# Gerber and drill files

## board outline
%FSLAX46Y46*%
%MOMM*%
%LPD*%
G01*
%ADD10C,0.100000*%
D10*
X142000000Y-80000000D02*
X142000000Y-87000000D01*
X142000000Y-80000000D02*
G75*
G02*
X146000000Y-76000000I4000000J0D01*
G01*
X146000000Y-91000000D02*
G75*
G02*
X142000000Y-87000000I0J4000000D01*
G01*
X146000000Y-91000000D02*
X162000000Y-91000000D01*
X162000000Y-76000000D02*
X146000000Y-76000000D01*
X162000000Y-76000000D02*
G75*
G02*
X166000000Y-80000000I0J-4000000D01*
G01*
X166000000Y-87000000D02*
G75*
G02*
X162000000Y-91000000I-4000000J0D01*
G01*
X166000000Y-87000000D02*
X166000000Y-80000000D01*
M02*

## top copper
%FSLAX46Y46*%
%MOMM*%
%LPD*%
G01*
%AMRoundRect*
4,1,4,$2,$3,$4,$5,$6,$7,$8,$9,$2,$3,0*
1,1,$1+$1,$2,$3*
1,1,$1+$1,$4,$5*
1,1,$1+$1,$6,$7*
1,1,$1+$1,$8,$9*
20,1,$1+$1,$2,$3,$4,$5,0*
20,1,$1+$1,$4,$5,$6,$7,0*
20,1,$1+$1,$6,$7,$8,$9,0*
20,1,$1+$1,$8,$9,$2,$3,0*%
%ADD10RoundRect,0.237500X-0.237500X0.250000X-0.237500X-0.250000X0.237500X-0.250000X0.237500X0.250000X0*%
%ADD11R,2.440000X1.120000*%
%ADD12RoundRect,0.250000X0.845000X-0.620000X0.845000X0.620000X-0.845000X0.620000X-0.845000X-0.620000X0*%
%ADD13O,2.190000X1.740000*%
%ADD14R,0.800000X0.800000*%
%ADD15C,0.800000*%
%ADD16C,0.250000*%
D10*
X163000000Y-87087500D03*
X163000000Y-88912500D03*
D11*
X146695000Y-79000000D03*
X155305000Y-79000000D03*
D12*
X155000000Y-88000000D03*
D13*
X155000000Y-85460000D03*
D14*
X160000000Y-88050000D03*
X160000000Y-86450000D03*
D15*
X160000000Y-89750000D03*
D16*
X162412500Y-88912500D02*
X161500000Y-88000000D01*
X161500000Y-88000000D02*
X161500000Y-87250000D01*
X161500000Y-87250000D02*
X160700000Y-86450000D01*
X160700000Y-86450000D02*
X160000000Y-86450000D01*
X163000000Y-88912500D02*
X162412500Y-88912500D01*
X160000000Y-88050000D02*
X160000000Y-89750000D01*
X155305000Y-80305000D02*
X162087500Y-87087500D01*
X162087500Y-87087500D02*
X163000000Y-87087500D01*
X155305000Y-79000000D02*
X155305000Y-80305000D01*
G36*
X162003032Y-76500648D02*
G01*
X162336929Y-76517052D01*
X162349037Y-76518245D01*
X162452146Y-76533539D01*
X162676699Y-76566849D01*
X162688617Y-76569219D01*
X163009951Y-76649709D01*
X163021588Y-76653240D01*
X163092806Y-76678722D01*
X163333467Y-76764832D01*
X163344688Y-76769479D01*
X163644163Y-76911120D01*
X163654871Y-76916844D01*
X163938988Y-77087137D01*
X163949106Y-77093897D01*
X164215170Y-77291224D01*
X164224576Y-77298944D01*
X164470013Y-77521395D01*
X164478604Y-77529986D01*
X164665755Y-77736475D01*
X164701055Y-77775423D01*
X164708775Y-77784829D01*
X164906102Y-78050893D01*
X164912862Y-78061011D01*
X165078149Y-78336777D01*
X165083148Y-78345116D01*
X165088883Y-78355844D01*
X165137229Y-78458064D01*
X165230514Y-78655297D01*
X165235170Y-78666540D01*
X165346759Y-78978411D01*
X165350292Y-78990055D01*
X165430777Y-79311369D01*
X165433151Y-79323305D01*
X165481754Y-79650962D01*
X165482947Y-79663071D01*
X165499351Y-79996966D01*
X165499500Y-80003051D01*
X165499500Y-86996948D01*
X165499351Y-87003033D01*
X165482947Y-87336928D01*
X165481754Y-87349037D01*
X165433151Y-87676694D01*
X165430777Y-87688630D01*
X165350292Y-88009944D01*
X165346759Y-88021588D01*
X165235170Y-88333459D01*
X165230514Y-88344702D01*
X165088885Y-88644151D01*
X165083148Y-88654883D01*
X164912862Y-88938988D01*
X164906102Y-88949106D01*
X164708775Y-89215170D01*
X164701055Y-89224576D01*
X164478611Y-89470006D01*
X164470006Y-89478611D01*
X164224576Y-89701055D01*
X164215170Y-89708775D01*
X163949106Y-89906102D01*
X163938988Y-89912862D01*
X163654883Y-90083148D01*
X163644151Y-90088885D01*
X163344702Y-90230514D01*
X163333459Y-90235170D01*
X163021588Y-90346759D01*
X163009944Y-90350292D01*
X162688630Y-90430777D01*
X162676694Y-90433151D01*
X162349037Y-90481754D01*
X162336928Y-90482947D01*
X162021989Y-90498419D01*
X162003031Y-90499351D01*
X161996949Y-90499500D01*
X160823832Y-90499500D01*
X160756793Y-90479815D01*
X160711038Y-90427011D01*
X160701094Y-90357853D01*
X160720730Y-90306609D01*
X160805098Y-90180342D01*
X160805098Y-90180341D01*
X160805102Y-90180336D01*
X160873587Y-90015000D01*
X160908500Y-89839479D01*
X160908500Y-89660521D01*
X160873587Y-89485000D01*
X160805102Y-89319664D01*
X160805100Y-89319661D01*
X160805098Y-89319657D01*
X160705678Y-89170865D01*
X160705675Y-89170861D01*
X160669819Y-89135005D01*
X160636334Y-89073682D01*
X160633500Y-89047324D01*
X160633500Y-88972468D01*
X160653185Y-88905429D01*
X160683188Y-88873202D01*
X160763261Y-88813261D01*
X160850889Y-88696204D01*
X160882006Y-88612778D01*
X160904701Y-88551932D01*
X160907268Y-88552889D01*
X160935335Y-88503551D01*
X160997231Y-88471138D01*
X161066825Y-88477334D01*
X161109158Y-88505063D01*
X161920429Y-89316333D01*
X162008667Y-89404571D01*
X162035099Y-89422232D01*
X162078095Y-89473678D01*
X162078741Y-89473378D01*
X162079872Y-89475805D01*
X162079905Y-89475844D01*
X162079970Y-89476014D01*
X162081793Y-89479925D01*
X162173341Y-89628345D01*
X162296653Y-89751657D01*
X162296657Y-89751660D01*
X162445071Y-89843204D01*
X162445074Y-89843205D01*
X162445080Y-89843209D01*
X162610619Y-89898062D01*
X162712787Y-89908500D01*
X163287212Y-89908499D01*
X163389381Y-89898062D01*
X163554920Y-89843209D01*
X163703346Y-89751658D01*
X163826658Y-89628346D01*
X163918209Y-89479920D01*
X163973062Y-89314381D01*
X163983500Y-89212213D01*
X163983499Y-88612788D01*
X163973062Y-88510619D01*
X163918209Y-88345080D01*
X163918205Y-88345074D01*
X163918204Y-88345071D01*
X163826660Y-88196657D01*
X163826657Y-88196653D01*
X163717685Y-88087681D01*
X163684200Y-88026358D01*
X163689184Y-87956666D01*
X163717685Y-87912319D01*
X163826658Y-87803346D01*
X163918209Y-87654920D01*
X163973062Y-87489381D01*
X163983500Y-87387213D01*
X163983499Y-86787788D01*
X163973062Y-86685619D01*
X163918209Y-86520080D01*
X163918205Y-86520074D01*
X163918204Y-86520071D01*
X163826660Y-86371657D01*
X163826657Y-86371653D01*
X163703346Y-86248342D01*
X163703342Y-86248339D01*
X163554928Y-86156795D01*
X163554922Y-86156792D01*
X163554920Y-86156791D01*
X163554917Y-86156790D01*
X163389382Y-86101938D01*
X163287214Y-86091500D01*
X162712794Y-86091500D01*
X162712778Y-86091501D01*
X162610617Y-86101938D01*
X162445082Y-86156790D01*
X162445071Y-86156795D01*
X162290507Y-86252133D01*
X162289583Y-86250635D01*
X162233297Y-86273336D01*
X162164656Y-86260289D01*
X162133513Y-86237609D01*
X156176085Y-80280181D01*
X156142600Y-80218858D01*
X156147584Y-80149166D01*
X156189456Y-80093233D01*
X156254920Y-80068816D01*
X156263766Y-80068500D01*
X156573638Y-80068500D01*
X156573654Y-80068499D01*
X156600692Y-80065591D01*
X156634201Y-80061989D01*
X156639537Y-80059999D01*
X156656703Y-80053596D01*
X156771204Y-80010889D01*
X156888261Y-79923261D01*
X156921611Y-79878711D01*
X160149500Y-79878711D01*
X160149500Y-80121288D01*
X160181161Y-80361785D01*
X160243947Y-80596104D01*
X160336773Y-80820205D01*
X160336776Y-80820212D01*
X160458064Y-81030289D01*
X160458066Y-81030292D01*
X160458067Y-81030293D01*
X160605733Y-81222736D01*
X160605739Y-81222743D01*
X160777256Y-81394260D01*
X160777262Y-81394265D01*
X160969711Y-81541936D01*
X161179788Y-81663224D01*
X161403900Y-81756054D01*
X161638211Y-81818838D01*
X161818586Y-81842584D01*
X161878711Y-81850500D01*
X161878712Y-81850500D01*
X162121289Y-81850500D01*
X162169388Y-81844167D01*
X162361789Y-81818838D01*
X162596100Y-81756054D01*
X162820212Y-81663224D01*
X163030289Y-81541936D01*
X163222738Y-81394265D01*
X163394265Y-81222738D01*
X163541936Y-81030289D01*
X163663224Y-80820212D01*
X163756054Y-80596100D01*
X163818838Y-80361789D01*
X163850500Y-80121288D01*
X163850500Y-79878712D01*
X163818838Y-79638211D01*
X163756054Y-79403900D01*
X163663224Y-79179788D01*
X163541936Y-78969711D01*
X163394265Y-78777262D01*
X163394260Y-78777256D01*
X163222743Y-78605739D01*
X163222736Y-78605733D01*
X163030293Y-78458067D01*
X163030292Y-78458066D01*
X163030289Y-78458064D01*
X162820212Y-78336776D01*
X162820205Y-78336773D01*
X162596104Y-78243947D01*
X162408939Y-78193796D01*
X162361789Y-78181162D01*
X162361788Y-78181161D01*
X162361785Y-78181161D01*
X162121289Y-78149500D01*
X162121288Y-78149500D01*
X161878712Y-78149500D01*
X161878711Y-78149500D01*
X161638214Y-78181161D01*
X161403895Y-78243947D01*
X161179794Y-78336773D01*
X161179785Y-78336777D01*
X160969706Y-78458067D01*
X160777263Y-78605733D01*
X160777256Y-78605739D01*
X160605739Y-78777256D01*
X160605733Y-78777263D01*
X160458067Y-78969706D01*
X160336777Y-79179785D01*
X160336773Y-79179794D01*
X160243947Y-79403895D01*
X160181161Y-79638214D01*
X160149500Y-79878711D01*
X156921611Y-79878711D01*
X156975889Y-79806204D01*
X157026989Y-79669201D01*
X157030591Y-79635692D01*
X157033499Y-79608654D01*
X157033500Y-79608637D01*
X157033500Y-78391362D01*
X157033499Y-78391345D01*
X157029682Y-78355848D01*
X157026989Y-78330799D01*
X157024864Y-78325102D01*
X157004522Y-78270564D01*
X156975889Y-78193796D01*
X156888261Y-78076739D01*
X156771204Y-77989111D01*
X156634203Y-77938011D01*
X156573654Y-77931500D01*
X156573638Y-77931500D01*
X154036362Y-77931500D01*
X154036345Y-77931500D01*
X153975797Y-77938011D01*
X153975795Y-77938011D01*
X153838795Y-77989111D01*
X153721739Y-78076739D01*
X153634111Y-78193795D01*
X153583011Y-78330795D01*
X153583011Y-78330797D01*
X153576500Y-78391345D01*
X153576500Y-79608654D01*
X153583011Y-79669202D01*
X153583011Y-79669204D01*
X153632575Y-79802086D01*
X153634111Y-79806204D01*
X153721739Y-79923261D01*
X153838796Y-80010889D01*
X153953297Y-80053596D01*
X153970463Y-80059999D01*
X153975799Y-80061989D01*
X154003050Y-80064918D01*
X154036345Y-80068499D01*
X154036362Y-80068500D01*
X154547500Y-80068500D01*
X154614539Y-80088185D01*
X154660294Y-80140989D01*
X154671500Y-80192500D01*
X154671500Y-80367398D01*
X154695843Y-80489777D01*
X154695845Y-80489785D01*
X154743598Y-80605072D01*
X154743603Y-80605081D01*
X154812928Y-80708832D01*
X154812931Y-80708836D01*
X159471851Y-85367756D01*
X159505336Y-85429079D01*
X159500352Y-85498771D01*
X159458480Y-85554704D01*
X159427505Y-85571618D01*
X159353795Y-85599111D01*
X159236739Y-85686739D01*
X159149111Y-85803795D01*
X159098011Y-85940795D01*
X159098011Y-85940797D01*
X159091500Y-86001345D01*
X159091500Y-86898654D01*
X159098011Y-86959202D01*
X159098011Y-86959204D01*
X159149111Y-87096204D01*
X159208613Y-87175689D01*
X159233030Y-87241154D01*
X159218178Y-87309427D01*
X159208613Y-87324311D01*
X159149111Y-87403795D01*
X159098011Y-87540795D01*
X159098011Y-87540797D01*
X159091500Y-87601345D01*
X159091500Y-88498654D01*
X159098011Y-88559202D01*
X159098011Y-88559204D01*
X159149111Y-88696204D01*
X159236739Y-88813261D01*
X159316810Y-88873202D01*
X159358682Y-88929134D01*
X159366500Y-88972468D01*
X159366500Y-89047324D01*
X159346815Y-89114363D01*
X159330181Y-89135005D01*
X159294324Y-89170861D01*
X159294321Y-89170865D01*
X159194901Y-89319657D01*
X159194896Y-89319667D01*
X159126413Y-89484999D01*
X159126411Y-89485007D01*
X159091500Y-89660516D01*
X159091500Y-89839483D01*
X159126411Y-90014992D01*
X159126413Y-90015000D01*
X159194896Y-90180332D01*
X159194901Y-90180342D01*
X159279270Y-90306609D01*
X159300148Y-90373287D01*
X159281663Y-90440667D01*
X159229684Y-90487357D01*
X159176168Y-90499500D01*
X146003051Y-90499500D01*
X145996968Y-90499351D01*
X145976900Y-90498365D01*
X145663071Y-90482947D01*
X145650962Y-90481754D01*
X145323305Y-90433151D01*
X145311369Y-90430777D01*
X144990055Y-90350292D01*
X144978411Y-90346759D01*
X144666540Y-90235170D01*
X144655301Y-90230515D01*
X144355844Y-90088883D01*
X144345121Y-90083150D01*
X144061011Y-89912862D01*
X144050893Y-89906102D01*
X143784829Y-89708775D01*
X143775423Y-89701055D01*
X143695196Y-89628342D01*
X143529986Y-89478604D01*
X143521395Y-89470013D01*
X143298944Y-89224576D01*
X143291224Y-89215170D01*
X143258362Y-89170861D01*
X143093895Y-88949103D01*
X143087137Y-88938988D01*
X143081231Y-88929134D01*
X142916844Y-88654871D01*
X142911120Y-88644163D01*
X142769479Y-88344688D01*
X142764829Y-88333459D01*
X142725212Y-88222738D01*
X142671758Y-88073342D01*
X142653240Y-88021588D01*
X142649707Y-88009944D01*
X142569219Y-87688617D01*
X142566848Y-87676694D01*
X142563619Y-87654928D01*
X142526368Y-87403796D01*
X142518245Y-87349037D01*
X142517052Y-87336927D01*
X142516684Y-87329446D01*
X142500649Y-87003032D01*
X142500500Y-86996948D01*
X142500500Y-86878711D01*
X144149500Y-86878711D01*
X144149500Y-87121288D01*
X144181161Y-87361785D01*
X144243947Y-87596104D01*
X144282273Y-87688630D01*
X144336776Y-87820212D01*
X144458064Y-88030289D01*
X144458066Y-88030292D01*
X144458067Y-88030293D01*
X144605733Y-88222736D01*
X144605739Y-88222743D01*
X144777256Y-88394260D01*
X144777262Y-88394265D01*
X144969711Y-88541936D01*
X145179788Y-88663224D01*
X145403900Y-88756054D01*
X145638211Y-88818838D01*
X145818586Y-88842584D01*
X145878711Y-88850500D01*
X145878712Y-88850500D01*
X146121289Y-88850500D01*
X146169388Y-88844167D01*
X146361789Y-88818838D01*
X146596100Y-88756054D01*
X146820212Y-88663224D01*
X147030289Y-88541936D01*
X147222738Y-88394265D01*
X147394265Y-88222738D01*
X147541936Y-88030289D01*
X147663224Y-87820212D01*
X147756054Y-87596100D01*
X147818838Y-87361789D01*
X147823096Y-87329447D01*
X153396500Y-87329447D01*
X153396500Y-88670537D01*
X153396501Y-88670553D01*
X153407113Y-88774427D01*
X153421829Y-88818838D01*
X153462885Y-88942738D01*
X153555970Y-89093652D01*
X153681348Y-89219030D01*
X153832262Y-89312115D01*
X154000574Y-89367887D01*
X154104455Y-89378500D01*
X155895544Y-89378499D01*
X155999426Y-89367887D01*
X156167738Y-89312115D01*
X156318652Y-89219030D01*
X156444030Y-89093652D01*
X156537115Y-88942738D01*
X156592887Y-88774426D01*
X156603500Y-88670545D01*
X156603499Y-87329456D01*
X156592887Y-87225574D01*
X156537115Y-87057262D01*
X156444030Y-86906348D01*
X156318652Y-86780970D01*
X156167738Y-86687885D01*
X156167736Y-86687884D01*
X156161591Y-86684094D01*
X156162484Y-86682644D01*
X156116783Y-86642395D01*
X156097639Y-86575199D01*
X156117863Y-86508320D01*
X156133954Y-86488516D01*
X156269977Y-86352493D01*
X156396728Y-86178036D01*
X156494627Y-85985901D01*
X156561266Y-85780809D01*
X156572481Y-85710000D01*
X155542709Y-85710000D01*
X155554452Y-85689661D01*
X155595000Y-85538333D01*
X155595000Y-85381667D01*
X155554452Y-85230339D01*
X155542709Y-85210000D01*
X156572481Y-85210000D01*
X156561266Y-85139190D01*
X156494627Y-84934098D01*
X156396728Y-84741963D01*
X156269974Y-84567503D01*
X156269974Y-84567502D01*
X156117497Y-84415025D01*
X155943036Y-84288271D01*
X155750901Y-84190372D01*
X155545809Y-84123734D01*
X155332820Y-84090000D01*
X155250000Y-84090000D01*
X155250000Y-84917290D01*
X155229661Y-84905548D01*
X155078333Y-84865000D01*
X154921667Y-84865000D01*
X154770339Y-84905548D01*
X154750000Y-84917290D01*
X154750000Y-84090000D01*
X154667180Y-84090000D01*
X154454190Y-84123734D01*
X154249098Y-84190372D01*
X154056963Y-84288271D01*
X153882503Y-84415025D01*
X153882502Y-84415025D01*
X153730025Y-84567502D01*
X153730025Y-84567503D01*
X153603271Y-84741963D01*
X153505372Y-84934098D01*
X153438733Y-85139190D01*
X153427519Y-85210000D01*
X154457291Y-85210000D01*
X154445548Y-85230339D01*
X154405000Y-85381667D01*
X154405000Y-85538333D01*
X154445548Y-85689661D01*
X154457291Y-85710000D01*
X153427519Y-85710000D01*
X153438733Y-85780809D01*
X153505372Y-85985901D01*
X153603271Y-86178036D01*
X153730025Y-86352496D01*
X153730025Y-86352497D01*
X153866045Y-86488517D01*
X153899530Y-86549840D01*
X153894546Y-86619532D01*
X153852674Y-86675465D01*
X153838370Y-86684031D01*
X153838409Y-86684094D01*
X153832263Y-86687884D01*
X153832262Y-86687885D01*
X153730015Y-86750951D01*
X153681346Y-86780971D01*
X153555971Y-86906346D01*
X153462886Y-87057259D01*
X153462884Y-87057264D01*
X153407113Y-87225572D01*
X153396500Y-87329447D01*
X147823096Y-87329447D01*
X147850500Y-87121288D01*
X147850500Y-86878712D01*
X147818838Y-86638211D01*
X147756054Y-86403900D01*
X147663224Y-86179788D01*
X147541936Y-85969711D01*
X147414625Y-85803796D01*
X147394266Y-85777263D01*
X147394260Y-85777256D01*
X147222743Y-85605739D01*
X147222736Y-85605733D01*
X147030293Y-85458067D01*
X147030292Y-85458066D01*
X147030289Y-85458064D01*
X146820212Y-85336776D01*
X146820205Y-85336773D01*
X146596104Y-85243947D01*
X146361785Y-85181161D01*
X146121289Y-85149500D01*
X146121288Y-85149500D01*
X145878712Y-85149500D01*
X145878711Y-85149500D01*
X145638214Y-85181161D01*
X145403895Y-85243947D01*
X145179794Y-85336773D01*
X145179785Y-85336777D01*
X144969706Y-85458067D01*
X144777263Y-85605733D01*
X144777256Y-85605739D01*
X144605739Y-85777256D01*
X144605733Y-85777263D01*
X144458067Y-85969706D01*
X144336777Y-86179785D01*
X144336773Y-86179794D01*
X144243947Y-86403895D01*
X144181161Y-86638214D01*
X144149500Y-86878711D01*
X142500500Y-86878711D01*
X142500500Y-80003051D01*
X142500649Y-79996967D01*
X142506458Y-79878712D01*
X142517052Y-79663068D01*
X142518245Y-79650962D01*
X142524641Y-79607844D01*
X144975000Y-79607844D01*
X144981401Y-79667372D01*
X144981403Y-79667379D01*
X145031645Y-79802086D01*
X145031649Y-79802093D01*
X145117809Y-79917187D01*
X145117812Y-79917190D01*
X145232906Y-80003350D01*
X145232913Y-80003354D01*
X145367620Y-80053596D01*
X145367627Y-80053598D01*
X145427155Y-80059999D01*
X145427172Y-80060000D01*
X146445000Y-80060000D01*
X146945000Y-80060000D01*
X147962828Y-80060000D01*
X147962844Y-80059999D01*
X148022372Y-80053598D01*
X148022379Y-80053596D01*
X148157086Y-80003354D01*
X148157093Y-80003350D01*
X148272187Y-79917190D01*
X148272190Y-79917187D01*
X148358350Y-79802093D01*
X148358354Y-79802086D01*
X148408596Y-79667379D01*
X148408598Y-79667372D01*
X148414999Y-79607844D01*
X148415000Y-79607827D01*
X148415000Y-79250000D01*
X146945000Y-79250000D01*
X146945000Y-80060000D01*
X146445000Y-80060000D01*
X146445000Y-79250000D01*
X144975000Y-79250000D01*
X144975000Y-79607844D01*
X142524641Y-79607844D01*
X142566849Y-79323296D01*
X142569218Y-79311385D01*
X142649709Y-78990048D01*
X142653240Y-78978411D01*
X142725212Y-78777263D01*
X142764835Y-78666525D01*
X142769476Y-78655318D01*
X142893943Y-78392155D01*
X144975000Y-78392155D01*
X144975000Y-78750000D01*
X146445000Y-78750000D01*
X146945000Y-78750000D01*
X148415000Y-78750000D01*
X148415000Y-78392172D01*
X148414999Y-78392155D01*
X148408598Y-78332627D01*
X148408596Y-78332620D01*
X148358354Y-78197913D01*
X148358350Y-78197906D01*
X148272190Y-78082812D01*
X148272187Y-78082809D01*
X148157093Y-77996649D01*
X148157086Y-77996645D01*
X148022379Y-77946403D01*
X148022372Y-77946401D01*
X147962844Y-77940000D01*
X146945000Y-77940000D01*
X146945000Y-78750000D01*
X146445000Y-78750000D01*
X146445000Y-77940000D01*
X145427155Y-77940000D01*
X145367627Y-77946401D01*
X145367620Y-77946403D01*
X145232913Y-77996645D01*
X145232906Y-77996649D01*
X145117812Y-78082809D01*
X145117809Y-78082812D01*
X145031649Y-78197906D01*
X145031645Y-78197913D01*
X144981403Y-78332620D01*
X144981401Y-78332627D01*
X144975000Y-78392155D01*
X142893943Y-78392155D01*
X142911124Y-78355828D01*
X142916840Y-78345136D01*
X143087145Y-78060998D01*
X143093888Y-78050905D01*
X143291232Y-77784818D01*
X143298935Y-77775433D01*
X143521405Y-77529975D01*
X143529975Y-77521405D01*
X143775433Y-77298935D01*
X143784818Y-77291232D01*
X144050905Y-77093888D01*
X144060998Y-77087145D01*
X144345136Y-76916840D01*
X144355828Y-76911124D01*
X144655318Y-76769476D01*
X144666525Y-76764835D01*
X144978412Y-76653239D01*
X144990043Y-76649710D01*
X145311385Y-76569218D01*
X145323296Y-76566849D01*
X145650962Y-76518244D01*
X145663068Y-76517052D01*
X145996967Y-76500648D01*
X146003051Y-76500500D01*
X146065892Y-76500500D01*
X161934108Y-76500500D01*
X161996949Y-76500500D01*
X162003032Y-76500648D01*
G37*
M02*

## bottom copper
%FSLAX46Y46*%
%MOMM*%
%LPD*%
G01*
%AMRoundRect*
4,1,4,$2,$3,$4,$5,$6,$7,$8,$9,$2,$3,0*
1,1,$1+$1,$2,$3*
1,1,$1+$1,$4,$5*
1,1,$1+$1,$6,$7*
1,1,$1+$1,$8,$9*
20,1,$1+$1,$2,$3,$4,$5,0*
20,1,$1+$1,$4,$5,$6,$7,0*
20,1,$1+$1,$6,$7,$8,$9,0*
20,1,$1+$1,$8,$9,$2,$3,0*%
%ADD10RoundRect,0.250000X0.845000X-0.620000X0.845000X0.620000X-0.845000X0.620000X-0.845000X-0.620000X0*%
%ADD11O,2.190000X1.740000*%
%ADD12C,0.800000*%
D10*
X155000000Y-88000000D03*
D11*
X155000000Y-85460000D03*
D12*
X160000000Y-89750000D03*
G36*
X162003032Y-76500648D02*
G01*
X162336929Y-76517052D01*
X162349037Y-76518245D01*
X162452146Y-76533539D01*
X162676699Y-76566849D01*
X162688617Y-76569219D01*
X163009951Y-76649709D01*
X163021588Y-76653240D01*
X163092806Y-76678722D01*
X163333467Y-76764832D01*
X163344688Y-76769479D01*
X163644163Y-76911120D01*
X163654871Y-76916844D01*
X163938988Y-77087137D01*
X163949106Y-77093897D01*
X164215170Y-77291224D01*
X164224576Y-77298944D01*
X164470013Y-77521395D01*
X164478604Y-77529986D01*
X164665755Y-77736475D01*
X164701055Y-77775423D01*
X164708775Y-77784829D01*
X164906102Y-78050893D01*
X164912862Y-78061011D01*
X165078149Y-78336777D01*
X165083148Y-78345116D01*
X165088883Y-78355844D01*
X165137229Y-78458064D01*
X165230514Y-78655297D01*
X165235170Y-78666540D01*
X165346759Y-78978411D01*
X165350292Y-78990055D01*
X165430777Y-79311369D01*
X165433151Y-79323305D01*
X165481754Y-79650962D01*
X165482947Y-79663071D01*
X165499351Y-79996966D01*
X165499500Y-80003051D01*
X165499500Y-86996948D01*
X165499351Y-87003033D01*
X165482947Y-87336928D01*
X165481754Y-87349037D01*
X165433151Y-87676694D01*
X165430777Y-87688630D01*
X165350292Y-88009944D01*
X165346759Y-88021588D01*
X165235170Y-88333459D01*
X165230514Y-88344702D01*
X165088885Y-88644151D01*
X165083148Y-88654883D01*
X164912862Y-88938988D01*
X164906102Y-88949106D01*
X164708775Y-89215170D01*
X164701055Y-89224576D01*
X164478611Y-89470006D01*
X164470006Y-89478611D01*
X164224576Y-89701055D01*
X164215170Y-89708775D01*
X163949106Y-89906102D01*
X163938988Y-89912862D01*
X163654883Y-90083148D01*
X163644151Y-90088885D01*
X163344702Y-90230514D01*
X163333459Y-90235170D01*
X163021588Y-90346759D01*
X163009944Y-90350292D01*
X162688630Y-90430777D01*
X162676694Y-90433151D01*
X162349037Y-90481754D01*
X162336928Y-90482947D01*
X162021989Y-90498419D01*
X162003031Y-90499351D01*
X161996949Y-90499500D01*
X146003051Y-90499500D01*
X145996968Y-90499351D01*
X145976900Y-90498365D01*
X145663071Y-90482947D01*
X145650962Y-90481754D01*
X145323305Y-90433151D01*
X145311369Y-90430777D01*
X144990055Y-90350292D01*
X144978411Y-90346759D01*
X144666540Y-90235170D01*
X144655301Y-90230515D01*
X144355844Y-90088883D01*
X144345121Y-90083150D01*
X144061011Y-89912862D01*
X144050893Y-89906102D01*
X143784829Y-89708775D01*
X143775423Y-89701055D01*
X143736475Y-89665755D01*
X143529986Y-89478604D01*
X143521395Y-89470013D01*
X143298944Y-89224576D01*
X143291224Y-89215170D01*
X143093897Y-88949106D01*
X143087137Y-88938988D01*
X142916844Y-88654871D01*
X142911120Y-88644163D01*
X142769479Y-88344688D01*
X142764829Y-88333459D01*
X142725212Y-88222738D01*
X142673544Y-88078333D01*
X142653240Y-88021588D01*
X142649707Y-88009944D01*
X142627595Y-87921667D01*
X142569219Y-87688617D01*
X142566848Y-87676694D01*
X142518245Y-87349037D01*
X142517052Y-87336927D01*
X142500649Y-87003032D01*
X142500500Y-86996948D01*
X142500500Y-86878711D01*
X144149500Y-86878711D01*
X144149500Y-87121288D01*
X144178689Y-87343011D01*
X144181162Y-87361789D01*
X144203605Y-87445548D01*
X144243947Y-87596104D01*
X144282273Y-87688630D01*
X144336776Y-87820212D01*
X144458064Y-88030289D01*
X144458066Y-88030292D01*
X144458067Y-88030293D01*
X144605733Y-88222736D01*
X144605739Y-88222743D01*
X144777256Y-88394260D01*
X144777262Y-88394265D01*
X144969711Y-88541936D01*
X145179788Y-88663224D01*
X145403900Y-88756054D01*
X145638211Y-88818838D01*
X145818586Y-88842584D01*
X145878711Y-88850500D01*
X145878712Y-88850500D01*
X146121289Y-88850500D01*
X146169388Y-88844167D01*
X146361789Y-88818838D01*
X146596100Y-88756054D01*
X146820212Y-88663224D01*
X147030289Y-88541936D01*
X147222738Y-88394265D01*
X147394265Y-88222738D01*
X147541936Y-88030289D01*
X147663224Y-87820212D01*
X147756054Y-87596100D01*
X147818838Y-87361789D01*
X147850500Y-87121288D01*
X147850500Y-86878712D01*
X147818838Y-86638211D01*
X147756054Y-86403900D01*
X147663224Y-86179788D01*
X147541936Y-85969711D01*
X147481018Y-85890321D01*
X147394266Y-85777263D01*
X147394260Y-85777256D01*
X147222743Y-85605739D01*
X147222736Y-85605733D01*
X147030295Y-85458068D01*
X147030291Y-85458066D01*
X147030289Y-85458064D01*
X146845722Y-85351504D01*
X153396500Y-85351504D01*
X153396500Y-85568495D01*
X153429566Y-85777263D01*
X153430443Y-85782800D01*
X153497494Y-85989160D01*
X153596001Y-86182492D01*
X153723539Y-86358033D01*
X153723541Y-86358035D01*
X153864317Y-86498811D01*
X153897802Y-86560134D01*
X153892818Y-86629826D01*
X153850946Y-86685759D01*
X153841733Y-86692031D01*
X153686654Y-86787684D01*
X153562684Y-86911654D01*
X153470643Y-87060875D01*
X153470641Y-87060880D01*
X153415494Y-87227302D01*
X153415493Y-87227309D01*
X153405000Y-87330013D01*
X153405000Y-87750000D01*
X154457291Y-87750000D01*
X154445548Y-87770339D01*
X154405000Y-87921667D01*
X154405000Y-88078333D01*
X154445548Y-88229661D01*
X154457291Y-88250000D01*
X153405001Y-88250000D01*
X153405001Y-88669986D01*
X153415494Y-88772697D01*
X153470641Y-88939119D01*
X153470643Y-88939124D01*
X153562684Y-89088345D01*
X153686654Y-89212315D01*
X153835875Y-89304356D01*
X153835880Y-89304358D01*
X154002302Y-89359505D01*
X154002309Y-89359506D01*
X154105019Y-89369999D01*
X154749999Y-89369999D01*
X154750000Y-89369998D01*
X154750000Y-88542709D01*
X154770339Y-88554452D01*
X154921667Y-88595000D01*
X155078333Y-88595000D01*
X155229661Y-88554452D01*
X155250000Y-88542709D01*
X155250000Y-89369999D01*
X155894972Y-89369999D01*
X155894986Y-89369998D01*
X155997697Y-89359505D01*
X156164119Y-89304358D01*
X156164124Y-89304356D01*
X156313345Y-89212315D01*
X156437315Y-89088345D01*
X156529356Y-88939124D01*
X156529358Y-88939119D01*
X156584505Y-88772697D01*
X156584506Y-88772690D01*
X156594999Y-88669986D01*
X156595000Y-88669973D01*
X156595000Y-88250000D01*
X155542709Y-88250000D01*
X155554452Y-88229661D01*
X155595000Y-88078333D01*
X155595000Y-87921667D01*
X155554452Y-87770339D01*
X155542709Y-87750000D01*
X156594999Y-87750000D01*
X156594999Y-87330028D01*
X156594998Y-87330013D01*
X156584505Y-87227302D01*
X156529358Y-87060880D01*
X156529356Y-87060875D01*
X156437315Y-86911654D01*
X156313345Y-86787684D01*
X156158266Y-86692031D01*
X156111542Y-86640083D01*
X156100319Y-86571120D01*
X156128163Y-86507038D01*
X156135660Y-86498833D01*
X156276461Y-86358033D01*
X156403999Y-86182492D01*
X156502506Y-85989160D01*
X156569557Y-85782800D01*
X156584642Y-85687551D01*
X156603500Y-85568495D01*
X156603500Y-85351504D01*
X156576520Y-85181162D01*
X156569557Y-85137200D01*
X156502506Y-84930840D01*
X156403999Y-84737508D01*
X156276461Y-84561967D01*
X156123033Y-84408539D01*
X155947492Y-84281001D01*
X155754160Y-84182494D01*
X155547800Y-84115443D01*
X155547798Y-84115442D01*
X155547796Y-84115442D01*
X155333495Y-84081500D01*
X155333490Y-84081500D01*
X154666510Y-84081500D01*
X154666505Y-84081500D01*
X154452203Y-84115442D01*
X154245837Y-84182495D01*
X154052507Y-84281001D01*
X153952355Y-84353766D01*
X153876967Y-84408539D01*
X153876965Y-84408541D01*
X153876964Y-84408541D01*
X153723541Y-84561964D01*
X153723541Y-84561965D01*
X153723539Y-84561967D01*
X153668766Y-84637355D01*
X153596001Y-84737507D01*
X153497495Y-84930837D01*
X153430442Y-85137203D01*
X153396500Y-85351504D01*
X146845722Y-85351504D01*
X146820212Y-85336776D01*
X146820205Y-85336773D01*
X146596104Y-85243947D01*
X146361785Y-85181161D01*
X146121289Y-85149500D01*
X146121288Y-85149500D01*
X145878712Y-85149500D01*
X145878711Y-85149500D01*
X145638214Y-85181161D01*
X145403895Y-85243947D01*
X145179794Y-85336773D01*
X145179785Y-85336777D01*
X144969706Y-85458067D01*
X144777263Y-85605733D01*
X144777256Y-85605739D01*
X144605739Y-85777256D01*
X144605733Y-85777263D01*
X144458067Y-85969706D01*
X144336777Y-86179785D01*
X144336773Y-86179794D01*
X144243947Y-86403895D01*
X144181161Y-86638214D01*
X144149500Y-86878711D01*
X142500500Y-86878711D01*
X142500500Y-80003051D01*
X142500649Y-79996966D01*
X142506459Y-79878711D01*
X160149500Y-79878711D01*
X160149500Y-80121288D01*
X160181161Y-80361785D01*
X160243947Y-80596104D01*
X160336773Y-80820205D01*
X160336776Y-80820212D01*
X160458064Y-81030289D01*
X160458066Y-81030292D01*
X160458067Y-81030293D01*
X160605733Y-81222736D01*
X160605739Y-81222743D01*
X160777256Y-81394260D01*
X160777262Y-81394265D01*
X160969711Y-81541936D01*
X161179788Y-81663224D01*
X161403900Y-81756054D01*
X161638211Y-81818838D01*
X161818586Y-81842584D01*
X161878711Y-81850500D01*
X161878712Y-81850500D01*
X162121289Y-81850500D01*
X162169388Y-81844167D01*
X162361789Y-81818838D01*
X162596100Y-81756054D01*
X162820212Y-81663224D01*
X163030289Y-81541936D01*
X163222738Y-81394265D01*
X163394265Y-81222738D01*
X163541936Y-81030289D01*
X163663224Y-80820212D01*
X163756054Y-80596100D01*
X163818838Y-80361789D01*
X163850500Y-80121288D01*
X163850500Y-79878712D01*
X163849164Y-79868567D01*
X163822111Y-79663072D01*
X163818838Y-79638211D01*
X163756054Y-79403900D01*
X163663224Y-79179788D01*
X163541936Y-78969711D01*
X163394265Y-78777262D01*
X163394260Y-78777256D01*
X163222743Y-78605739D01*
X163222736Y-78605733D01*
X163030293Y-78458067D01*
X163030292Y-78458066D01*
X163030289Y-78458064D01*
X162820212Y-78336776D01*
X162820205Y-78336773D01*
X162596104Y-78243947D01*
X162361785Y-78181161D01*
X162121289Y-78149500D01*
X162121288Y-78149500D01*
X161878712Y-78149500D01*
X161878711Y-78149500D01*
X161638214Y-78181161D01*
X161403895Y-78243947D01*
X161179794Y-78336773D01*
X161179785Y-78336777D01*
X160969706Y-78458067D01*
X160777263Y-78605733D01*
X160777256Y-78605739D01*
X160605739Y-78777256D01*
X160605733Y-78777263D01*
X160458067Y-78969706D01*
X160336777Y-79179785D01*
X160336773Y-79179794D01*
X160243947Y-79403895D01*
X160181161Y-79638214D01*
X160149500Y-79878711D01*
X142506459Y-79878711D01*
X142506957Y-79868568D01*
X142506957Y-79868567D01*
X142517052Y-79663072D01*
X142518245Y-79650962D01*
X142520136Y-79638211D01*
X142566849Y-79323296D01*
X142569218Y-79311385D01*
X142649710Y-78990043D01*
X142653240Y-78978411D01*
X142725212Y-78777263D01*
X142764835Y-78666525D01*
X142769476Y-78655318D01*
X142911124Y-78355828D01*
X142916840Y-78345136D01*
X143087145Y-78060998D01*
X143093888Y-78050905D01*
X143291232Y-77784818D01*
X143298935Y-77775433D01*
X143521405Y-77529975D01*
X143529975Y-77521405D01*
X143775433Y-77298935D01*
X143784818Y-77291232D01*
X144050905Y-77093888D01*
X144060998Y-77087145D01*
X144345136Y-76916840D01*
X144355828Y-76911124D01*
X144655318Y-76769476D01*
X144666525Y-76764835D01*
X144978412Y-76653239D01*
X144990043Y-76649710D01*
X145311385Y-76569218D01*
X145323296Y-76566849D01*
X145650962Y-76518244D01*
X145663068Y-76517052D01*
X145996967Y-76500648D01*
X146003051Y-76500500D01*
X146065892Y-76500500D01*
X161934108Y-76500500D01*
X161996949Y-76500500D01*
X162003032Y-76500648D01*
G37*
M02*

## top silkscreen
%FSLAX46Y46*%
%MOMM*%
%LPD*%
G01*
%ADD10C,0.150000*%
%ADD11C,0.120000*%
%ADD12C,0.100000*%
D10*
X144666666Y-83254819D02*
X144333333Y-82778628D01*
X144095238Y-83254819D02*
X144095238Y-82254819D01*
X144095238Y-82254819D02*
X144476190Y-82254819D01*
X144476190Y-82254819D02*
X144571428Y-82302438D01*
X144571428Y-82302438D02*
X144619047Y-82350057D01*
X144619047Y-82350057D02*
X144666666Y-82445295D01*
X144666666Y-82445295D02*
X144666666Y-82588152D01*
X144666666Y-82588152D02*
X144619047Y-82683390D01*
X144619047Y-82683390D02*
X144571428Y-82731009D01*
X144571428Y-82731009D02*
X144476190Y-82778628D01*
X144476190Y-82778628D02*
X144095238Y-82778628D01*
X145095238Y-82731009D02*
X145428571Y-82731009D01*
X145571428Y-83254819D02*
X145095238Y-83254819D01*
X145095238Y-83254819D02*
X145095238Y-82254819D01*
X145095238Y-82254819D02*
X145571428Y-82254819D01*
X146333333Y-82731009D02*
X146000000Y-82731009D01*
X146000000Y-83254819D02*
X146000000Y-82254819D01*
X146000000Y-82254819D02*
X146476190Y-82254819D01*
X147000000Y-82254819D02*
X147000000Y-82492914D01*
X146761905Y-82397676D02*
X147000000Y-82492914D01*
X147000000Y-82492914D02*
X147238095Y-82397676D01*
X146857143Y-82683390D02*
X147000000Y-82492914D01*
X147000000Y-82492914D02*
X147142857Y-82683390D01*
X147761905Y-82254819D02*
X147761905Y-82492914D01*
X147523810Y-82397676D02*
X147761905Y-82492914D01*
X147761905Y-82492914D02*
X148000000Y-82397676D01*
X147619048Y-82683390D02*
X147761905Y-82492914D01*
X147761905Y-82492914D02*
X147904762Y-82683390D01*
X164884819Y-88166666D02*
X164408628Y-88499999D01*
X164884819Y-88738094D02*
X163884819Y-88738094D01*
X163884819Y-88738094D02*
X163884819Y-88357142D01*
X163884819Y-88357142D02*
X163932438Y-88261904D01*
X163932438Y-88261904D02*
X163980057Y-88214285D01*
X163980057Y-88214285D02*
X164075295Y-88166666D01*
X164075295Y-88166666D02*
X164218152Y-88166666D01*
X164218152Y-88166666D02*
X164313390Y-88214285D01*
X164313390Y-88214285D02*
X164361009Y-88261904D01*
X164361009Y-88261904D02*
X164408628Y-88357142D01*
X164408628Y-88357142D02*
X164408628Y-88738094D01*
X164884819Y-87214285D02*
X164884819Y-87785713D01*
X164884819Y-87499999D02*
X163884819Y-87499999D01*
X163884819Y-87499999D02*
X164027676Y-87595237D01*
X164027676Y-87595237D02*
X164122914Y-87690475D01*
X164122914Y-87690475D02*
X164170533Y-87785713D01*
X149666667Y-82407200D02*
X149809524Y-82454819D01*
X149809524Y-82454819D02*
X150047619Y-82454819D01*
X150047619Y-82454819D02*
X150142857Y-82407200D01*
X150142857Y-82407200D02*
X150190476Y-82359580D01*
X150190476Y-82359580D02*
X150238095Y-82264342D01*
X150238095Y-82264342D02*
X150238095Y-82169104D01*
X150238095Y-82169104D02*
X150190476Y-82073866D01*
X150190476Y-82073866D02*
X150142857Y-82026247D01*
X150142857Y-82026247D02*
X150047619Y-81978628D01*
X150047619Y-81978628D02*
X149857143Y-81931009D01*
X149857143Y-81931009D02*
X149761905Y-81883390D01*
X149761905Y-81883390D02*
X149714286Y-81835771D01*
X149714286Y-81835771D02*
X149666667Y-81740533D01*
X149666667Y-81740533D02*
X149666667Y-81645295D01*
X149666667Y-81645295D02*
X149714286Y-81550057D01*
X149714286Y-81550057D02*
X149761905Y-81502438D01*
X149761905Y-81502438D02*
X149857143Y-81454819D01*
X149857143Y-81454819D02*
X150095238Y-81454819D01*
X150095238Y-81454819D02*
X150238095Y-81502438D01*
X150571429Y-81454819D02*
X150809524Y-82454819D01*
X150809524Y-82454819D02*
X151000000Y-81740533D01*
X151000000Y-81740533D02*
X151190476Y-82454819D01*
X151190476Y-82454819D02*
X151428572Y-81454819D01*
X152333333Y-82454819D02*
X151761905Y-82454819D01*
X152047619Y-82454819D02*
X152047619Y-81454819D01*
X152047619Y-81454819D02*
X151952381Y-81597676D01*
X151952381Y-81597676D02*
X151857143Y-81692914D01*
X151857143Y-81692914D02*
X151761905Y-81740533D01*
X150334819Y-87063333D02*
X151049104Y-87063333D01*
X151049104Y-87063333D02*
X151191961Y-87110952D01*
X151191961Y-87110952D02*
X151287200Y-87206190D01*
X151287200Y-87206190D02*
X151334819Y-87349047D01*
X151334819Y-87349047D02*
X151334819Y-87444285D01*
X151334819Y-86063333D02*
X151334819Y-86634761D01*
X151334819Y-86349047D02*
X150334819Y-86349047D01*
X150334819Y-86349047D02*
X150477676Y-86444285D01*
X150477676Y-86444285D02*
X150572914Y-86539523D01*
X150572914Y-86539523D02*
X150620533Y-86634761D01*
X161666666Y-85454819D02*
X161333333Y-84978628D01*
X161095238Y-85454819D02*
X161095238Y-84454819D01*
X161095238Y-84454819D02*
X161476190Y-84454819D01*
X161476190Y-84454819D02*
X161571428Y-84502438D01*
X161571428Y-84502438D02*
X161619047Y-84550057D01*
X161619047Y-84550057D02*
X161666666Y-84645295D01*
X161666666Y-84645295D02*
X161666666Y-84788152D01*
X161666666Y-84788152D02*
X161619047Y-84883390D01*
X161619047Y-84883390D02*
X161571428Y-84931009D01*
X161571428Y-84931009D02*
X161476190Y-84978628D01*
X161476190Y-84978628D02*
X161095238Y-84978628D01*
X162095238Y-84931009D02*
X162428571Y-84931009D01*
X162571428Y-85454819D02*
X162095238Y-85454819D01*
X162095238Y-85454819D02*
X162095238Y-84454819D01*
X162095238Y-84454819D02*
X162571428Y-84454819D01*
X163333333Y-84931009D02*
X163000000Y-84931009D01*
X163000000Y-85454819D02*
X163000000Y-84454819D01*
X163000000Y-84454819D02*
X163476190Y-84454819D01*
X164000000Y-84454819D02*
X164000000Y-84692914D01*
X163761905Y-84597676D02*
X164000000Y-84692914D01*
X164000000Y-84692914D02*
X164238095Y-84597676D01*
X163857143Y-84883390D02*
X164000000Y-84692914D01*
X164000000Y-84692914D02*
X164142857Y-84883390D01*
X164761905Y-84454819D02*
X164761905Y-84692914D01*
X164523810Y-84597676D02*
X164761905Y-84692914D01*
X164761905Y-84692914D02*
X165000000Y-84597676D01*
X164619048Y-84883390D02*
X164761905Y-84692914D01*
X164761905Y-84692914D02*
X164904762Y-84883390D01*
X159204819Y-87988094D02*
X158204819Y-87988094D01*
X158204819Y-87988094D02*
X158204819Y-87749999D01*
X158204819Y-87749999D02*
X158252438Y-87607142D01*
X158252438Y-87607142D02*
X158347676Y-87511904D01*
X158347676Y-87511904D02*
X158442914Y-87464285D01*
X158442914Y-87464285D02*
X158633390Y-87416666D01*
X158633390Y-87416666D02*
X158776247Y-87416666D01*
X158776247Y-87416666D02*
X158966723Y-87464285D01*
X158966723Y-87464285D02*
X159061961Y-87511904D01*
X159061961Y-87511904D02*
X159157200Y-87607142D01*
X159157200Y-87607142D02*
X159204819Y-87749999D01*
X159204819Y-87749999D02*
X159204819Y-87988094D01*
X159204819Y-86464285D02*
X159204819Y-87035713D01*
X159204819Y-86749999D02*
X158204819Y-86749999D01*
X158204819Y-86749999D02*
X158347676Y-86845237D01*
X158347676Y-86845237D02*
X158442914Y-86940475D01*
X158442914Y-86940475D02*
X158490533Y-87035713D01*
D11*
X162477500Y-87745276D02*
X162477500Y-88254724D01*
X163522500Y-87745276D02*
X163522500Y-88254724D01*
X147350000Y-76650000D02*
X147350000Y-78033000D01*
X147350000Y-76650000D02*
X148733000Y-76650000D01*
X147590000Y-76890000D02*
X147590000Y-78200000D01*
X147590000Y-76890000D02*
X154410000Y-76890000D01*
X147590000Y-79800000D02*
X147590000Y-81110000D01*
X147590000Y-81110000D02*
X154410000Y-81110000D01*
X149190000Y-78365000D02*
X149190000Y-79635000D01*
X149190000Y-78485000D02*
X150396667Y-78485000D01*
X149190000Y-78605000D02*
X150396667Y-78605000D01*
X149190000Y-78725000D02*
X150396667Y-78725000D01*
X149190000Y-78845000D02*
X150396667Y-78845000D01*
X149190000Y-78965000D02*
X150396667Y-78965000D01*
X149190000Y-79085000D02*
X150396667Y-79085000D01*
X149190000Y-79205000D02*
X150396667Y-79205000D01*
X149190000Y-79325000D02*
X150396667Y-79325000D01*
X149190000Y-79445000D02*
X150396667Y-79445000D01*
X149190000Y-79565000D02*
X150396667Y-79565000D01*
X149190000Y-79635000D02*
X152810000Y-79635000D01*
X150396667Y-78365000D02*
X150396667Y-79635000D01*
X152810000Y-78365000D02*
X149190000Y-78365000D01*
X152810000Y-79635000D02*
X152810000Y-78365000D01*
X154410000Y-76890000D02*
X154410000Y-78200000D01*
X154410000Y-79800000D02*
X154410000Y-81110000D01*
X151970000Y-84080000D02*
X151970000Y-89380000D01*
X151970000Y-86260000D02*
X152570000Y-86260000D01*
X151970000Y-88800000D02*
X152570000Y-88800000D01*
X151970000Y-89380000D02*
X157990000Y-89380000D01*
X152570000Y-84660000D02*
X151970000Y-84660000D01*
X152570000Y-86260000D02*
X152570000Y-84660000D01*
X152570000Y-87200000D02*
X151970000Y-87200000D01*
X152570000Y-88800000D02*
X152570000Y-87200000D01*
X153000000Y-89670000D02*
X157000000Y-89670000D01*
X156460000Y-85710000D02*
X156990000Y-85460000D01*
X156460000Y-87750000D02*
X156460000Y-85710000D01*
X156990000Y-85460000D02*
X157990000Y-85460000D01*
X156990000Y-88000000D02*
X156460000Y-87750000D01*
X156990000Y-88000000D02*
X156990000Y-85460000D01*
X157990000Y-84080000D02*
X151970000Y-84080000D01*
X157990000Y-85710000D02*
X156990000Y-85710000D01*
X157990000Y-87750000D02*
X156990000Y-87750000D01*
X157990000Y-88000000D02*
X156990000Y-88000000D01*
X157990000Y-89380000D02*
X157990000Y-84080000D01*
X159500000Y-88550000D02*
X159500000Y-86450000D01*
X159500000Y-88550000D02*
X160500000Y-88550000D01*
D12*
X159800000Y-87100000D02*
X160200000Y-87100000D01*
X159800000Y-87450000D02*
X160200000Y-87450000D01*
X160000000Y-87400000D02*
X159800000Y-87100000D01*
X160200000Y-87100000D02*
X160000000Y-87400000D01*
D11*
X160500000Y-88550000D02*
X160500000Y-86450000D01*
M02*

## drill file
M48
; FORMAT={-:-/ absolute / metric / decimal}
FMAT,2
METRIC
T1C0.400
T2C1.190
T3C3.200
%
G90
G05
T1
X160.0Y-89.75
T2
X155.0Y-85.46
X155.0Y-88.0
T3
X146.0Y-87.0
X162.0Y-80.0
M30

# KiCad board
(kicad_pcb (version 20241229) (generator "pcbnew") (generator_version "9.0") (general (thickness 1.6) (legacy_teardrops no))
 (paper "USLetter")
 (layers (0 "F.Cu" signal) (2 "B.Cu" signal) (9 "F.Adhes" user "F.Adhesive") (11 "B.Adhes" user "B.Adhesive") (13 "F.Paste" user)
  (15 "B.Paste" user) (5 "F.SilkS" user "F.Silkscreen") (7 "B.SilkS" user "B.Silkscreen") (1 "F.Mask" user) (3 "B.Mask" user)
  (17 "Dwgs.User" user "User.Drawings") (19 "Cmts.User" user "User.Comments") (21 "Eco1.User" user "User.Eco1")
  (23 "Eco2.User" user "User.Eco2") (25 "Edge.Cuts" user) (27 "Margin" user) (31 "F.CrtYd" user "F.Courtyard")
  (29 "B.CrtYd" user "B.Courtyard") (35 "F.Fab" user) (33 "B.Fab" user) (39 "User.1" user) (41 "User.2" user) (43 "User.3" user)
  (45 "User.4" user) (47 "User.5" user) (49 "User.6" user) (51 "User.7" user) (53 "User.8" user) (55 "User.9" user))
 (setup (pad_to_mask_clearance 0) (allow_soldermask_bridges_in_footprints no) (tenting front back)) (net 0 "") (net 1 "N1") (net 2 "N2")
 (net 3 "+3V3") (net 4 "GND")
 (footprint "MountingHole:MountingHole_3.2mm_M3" (layer "F.Cu") (at 146 87)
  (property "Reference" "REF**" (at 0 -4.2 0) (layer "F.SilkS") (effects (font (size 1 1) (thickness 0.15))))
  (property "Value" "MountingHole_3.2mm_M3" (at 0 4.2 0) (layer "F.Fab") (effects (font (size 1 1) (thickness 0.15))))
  (pad "" np_thru_hole circle (at 0 0) (size 3.2 3.2) (drill 3.2) (layers "*.Cu" "*.Mask")))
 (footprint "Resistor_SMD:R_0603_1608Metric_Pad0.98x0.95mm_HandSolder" (layer "F.Cu") (at 163 88 -90)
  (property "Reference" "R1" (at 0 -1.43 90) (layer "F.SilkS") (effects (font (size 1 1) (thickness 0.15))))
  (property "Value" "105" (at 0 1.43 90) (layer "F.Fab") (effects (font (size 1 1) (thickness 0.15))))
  (fp_line (start -0.254724 0.5225) (end 0.254724 0.5225) (stroke (width 0.12) (type solid)) (layer "F.SilkS"))
  (fp_line (start -0.254724 -0.5225) (end 0.254724 -0.5225) (stroke (width 0.12) (type solid)) (layer "F.SilkS"))
  (pad "1" smd roundrect (at -0.9125 0 270) (size 0.975 0.95) (layers "F.Cu" "F.Mask" "F.Paste") (roundrect_rratio 0.25) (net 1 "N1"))
  (pad "2" smd roundrect (at 0.9125 0 270) (size 0.975 0.95) (layers "F.Cu" "F.Mask" "F.Paste") (roundrect_rratio 0.25) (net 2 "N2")))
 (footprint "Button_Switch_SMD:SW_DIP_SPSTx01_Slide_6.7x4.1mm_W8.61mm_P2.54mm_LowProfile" (layer "F.Cu") (at 151 79)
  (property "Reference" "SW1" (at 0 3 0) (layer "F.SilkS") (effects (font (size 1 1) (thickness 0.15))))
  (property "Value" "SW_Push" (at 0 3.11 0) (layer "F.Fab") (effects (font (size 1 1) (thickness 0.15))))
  (fp_line (start -3.65 -2.35) (end -3.65 -0.967) (stroke (width 0.12) (type solid)) (layer "F.SilkS"))
  (fp_line (start -3.65 -2.35) (end -2.267 -2.35) (stroke (width 0.12) (type solid)) (layer "F.SilkS"))
  (fp_line (start -3.41 -2.11) (end -3.41 -0.8) (stroke (width 0.12) (type solid)) (layer "F.SilkS"))
  (fp_line (start -3.41 -2.11) (end 3.41 -2.11) (stroke (width 0.12) (type solid)) (layer "F.SilkS"))
  (fp_line (start -3.41 0.8) (end -3.41 2.11) (stroke (width 0.12) (type solid)) (layer "F.SilkS"))
  (fp_line (start -3.41 2.11) (end 3.41 2.11) (stroke (width 0.12) (type solid)) (layer "F.SilkS"))
  (fp_line (start -1.81 -0.635) (end -1.81 0.635) (stroke (width 0.12) (type solid)) (layer "F.SilkS"))
  (fp_line (start -1.81 -0.515) (end -0.603333 -0.515) (stroke (width 0.12) (type solid)) (layer "F.SilkS"))
  (fp_line (start -1.81 -0.395) (end -0.603333 -0.395) (stroke (width 0.12) (type solid)) (layer "F.SilkS"))
  (fp_line (start -1.81 -0.275) (end -0.603333 -0.275) (stroke (width 0.12) (type solid)) (layer "F.SilkS"))
  (fp_line (start -1.81 -0.155) (end -0.603333 -0.155) (stroke (width 0.12) (type solid)) (layer "F.SilkS"))
  (fp_line (start -1.81 -0.035) (end -0.603333 -0.035) (stroke (width 0.12) (type solid)) (layer "F.SilkS"))
  (fp_line (start -1.81 0.085) (end -0.603333 0.085) (stroke (width 0.12) (type solid)) (layer "F.SilkS"))
  (fp_line (start -1.81 0.205) (end -0.603333 0.205) (stroke (width 0.12) (type solid)) (layer "F.SilkS"))
  (fp_line (start -1.81 0.325) (end -0.603333 0.325) (stroke (width 0.12) (type solid)) (layer "F.SilkS"))
  (fp_line (start -1.81 0.445) (end -0.603333 0.445) (stroke (width 0.12) (type solid)) (layer "F.SilkS"))
  (fp_line (start -1.81 0.565) (end -0.603333 0.565) (stroke (width 0.12) (type solid)) (layer "F.SilkS"))
  (fp_line (start -1.81 0.635) (end 1.81 0.635) (stroke (width 0.12) (type solid)) (layer "F.SilkS"))
  (fp_line (start -0.603333 -0.635) (end -0.603333 0.635) (stroke (width 0.12) (type solid)) (layer "F.SilkS"))
  (fp_line (start 1.81 -0.635) (end -1.81 -0.635) (stroke (width 0.12) (type solid)) (layer "F.SilkS"))
  (fp_line (start 1.81 0.635) (end 1.81 -0.635) (stroke (width 0.12) (type solid)) (layer "F.SilkS"))
  (fp_line (start 3.41 -2.11) (end 3.41 -0.8) (stroke (width 0.12) (type solid)) (layer "F.SilkS"))
  (fp_line (start 3.41 0.8) (end 3.41 2.11) (stroke (width 0.12) (type solid)) (layer "F.SilkS"))
  (pad "1" smd rect (at -4.305 0) (size 2.44 1.12) (layers "F.Cu" "F.Mask" "F.Paste") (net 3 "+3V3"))
  (pad "2" smd rect (at 4.305 0) (size 2.44 1.12) (layers "F.Cu" "F.Mask" "F.Paste") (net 1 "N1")))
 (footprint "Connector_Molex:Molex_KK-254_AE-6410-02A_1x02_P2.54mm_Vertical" (layer "F.Cu") (at 155 88 90)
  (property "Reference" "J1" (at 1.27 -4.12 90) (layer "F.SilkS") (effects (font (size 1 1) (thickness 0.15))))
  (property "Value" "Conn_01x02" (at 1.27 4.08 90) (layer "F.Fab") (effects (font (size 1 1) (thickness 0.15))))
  (fp_line (start 3.92 -3.03) (end -1.38 -3.03) (stroke (width 0.12) (type solid)) (layer "F.SilkS"))
  (fp_line (start 1.74 -3.03) (end 1.74 -2.43) (stroke (width 0.12) (type solid)) (layer "F.SilkS"))
  (fp_line (start -0.8 -3.03) (end -0.8 -2.43) (stroke (width 0.12) (type solid)) (layer "F.SilkS"))
  (fp_line (start -1.38 -3.03) (end -1.38 2.99) (stroke (width 0.12) (type solid)) (layer "F.SilkS"))
  (fp_line (start 3.34 -2.43) (end 3.34 -3.03) (stroke (width 0.12) (type solid)) (layer "F.SilkS"))
  (fp_line (start 1.74 -2.43) (end 3.34 -2.43) (stroke (width 0.12) (type solid)) (layer "F.SilkS"))
  (fp_line (start 0.8 -2.43) (end 0.8 -3.03) (stroke (width 0.12) (type solid)) (layer "F.SilkS"))
  (fp_line (start -0.8 -2.43) (end 0.8 -2.43) (stroke (width 0.12) (type solid)) (layer "F.SilkS"))
  (fp_line (start -1.67 -2) (end -1.67 2) (stroke (width 0.12) (type solid)) (layer "F.SilkS"))
  (fp_line (start 2.29 1.46) (end 2.54 1.99) (stroke (width 0.12) (type solid)) (layer "F.SilkS"))
  (fp_line (start 0.25 1.46) (end 2.29 1.46) (stroke (width 0.12) (type solid)) (layer "F.SilkS"))
  (fp_line (start 2.54 1.99) (end 2.54 2.99) (stroke (width 0.12) (type solid)) (layer "F.SilkS"))
  (fp_line (start 0 1.99) (end 0.25 1.46) (stroke (width 0.12) (type solid)) (layer "F.SilkS"))
  (fp_line (start 0 1.99) (end 2.54 1.99) (stroke (width 0.12) (type solid)) (layer "F.SilkS"))
  (fp_line (start 3.92 2.99) (end 3.92 -3.03) (stroke (width 0.12) (type solid)) (layer "F.SilkS"))
  (fp_line (start 2.29 2.99) (end 2.29 1.99) (stroke (width 0.12) (type solid)) (layer "F.SilkS"))
  (fp_line (start 0.25 2.99) (end 0.25 1.99) (stroke (width 0.12) (type solid)) (layer "F.SilkS"))
  (fp_line (start 0 2.99) (end 0 1.99) (stroke (width 0.12) (type solid)) (layer "F.SilkS"))
  (fp_line (start -1.38 2.99) (end 3.92 2.99) (stroke (width 0.12) (type solid)) (layer "F.SilkS"))
  (pad "1" thru_hole roundrect (at 0 0 90) (size 1.74 2.19) (drill 1.19) (layers "*.Cu" "*.Mask") (remove_unused_layers no)
   (roundrect_rratio 0.143678) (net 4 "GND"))
  (pad "2" thru_hole oval (at 2.54 0 90) (size 1.74 2.19) (drill 1.19) (layers "*.Cu" "*.Mask") (remove_unused_layers no) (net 3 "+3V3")))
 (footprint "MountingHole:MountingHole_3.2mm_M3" (layer "F.Cu") (at 162 80)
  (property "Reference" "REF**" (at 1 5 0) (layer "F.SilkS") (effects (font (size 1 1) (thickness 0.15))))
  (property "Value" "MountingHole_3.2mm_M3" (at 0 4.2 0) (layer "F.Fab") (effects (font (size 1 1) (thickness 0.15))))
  (pad "" np_thru_hole circle (at 0 0) (size 3.2 3.2) (drill 3.2) (layers "*.Cu" "*.Mask")))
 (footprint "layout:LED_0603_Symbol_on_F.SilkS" (layer "F.Cu") (at 160 87.25 90)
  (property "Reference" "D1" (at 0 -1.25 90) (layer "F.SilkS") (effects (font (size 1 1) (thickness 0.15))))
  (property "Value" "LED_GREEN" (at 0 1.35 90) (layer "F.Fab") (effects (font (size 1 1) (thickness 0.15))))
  (fp_line (start -1.3 -0.5) (end 0.8 -0.5) (stroke (width 0.12) (type solid)) (layer "F.SilkS"))
  (fp_line (start -1.3 -0.5) (end -1.3 0.5) (stroke (width 0.12) (type solid)) (layer "F.SilkS"))
  (fp_line (start 0.15 -0.2) (end 0.15 0.2) (stroke (width 0.1) (type solid)) (layer "F.SilkS"))
  (fp_line (start -0.2 -0.2) (end -0.2 0.2) (stroke (width 0.1) (type solid)) (layer "F.SilkS"))
  (fp_line (start -0.15 0) (end 0.15 -0.2) (stroke (width 0.1) (type solid)) (layer "F.SilkS"))
  (fp_line (start 0.15 0.2) (end -0.15 0) (stroke (width 0.1) (type solid)) (layer "F.SilkS"))
  (fp_line (start -1.3 0.5) (end 0.8 0.5) (stroke (width 0.12) (type solid)) (layer "F.SilkS"))
  (pad "1" smd rect (at -0.8 0 270) (size 0.8 0.8) (layers "F.Cu" "F.Mask" "F.Paste") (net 4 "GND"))
  (pad "2" smd rect (at 0.8 0 270) (size 0.8 0.8) (layers "F.Cu" "F.Mask" "F.Paste") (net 2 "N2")))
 (gr_line (start 142 80) (end 142 87) (stroke (width 0.1) (type default)) (layer "Edge.Cuts"))
 (gr_arc (start 142 80) (mid 143.171573 77.171573) (end 146 76) (stroke (width 0.1) (type default)) (layer "Edge.Cuts"))
 (gr_arc (start 146 91) (mid 143.171573 89.828427) (end 142 87) (stroke (width 0.1) (type default)) (layer "Edge.Cuts"))
 (gr_line (start 146 91) (end 162 91) (stroke (width 0.1) (type default)) (layer "Edge.Cuts"))
 (gr_line (start 162 76) (end 146 76) (stroke (width 0.1) (type default)) (layer "Edge.Cuts"))
 (gr_arc (start 162 76) (mid 164.828427 77.171573) (end 166 80) (stroke (width 0.1) (type default)) (layer "Edge.Cuts"))
 (gr_arc (start 166 87) (mid 164.828427 89.828427) (end 162 91) (stroke (width 0.1) (type default)) (layer "Edge.Cuts"))
 (gr_line (start 166 87) (end 166 80) (stroke (width 0.1) (type default)) (layer "Edge.Cuts"))
 (segment (start 162.4125 88.9125) (end 161.5 88) (width 0.25) (layer "F.Cu") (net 2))
 (segment (start 161.5 88) (end 161.5 87.25) (width 0.25) (layer "F.Cu") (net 2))
 (segment (start 161.5 87.25) (end 160.7 86.45) (width 0.25) (layer "F.Cu") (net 2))
 (segment (start 160.7 86.45) (end 160 86.45) (width 0.25) (layer "F.Cu") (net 2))
 (segment (start 163 88.9125) (end 162.4125 88.9125) (width 0.25) (layer "F.Cu") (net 2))
 (segment (start 160 88.05) (end 160 89.75) (width 0.25) (layer "F.Cu") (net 4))
 (via (at 160 89.75) (size 0.8) (drill 0.4) (layers "F.Cu" "B.Cu") (free yes) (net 4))
 (segment (start 155.305 80.305) (end 162.0875 87.0875) (width 0.25) (layer "F.Cu") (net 1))
 (segment (start 162.0875 87.0875) (end 163 87.0875) (width 0.25) (layer "F.Cu") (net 1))
 (segment (start 155.305 79) (end 155.305 80.305) (width 0.25) (layer "F.Cu") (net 1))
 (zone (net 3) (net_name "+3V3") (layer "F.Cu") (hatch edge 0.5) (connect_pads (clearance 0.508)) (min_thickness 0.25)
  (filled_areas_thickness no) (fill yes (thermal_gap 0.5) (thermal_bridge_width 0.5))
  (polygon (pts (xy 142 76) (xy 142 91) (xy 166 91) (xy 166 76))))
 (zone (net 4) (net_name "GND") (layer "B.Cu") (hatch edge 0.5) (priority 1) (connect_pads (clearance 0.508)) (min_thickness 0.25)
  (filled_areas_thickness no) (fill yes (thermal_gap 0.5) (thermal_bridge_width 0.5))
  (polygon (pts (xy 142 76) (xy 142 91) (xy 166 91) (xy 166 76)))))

